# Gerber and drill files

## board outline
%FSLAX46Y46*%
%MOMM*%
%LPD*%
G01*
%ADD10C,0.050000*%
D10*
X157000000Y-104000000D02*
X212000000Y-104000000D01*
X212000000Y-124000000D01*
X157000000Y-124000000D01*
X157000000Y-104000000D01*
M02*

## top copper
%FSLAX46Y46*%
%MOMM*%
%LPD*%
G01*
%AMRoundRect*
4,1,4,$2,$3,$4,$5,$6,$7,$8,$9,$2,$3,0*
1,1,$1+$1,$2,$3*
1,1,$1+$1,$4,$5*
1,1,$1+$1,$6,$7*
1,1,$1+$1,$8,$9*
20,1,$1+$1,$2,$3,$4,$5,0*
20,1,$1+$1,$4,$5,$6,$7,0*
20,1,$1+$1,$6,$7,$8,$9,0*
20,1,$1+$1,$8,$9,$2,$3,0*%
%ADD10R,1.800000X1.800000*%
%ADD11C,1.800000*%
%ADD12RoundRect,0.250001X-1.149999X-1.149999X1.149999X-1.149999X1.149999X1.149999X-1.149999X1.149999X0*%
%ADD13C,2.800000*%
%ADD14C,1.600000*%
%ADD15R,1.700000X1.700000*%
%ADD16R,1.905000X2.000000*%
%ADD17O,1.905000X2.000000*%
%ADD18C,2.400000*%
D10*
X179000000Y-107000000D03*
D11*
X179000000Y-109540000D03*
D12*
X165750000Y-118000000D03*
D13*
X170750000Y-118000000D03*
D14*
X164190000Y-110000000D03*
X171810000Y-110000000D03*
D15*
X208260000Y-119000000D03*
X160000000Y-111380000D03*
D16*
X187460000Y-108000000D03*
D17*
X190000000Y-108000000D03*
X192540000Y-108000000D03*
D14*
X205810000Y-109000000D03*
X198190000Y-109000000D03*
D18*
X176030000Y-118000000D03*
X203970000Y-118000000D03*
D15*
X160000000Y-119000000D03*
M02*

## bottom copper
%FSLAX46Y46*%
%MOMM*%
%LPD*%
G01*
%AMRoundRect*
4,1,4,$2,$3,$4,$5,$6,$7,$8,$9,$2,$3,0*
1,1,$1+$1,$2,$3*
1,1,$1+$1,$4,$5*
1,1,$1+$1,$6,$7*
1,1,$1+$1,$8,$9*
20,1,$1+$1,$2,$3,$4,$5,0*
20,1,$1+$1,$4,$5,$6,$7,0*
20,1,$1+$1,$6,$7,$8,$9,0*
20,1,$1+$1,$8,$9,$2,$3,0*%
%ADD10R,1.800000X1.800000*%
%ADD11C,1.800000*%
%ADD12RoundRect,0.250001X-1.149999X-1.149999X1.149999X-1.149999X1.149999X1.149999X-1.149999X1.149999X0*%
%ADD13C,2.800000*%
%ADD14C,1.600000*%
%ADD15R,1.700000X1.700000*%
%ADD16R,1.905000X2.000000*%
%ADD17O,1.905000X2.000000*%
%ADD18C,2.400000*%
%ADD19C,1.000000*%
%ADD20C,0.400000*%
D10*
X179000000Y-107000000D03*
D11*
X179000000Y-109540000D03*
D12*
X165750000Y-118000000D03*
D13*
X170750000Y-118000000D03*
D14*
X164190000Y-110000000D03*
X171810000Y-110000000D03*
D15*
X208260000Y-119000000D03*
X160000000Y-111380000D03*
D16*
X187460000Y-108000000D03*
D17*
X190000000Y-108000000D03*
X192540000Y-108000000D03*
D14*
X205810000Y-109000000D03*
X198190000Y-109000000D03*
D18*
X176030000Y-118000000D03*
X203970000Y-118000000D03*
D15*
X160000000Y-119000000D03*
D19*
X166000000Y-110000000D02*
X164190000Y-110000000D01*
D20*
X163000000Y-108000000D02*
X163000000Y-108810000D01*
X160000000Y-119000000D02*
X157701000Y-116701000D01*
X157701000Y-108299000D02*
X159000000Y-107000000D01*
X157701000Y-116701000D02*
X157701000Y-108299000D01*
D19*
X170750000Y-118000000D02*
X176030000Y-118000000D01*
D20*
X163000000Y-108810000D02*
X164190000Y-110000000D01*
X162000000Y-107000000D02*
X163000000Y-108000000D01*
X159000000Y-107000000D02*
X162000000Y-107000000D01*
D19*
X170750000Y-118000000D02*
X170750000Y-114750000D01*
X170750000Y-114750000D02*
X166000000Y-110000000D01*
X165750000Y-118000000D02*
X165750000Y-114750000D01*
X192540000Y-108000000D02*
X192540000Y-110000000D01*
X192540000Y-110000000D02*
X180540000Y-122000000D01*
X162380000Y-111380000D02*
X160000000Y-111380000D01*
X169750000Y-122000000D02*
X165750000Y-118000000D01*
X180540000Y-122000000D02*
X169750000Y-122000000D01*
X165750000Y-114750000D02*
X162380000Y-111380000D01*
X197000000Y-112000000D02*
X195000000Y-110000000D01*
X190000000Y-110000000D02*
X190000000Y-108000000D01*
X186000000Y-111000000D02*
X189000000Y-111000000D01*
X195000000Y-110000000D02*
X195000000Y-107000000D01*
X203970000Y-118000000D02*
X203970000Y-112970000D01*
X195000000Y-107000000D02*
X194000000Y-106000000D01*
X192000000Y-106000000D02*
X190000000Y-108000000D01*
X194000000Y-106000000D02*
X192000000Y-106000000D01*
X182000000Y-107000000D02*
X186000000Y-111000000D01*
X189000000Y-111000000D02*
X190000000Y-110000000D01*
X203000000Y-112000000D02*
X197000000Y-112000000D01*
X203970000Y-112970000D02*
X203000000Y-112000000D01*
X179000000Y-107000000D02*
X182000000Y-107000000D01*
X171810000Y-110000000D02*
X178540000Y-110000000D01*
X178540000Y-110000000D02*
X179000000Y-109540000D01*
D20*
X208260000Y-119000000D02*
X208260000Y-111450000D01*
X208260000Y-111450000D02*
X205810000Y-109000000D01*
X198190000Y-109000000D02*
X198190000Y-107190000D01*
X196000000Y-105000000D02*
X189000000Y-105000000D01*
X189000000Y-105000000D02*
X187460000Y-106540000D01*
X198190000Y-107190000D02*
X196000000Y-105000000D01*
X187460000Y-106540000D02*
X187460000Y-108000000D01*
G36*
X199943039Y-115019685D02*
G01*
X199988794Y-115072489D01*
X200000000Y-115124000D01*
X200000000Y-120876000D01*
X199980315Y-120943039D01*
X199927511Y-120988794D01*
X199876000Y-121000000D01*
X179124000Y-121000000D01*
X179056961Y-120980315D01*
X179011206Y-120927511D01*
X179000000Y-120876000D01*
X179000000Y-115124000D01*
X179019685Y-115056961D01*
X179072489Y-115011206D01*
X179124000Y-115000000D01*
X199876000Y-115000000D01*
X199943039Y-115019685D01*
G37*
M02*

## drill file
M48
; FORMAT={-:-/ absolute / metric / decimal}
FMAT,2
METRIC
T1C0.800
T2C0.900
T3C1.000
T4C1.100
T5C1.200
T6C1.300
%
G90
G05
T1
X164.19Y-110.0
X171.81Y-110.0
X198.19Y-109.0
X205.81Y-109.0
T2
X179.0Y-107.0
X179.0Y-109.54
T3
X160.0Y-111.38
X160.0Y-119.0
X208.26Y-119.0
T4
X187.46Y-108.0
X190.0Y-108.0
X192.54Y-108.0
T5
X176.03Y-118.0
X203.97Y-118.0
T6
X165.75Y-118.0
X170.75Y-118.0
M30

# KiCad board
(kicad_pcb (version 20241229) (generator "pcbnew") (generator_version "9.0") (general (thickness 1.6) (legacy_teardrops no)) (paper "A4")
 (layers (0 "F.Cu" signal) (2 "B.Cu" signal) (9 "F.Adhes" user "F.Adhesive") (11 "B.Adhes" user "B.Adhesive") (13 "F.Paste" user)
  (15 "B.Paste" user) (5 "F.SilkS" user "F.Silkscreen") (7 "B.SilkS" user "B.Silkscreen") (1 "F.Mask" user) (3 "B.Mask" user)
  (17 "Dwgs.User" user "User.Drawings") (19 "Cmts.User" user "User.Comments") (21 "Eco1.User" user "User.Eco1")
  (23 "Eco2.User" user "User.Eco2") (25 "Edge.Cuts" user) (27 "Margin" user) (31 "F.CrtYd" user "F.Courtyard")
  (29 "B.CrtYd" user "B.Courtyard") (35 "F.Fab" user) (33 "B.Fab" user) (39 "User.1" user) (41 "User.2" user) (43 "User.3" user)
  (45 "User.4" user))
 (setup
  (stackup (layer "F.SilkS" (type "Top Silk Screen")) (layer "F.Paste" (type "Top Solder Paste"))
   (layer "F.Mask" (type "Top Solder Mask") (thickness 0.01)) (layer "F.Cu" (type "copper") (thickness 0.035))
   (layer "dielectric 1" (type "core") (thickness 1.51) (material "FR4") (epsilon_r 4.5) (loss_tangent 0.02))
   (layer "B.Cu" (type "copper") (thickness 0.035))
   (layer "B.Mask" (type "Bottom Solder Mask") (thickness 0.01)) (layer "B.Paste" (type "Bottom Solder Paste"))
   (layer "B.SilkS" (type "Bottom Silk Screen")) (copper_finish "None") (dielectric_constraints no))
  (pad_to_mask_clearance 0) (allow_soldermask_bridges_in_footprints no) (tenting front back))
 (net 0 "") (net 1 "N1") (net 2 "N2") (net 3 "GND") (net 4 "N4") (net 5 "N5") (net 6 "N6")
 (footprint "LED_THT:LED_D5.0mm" (layer "F.Cu") (at 179 107 -90)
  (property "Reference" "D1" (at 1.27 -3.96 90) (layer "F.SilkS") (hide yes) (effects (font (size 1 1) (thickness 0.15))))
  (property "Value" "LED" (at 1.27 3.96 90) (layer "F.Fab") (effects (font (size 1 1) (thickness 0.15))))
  (pad "1" thru_hole rect (at 0 0 270) (size 1.8 1.8) (drill 0.9) (layers "*.Cu" "*.Mask") (remove_unused_layers no) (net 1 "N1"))
  (pad "2" thru_hole circle (at 2.54 0 270) (size 1.8 1.8) (drill 0.9) (layers "*.Cu" "*.Mask") (remove_unused_layers no) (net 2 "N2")))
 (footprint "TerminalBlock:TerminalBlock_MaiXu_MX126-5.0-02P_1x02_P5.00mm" (layer "F.Cu") (at 165.75 118)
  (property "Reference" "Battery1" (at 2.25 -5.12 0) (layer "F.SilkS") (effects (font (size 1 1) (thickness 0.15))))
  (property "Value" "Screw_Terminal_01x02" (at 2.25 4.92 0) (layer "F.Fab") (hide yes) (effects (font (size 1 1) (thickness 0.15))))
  (pad "1" thru_hole roundrect (at 0 0) (size 2.8 2.8) (drill 1.3) (layers "*.Cu" "*.Mask") (remove_unused_layers no)
   (roundrect_rratio 0.089286) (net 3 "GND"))
  (pad "2" thru_hole circle (at 5 0) (size 2.8 2.8) (drill 1.3) (layers "*.Cu" "*.Mask") (remove_unused_layers no) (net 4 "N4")))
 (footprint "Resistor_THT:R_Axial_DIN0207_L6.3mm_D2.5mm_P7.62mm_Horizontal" (layer "F.Cu") (at 164.19 110)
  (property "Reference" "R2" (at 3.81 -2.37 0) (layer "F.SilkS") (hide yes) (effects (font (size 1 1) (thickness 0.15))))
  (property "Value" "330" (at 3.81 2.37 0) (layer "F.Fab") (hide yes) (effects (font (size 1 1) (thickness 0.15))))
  (pad "1" thru_hole circle (at 0 0) (size 1.6 1.6) (drill 0.8) (layers "*.Cu" "*.Mask") (remove_unused_layers no) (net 4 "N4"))
  (pad "2" thru_hole circle (at 7.62 0) (size 1.6 1.6) (drill 0.8) (layers "*.Cu" "*.Mask") (remove_unused_layers no) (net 2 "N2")))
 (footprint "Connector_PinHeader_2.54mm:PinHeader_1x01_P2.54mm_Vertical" (layer "F.Cu") (at 208.26 119)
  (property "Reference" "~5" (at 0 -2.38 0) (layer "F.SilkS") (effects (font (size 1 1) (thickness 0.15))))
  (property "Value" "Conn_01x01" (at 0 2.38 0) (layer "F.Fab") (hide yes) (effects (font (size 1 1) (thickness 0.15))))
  (pad "1" thru_hole rect (at 0 0) (size 1.7 1.7) (drill 1) (layers "*.Cu" "*.Mask") (remove_unused_layers no) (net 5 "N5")))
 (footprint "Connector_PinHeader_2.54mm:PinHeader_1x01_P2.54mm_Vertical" (layer "F.Cu") (at 160 111.38)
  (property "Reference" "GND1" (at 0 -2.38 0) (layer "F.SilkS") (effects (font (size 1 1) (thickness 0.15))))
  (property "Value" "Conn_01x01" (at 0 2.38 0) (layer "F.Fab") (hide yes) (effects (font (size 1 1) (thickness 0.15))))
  (pad "1" thru_hole rect (at 0 0) (size 1.7 1.7) (drill 1) (layers "*.Cu" "*.Mask") (remove_unused_layers no) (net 3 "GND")))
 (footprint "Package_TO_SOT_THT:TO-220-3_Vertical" (layer "F.Cu") (at 187.46 108)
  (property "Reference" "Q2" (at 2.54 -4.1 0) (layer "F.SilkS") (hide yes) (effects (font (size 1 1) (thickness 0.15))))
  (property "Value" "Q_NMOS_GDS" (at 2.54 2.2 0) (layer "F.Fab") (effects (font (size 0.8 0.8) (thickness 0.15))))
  (pad "1" thru_hole rect (at 0 0) (size 1.905 2) (drill 1.1) (layers "*.Cu" "*.Mask") (remove_unused_layers no) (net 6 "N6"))
  (pad "2" thru_hole oval (at 2.54 0) (size 1.905 2) (drill 1.1) (layers "*.Cu" "*.Mask") (remove_unused_layers no) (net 1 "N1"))
  (pad "3" thru_hole oval (at 5.08 0) (size 1.905 2) (drill 1.1) (layers "*.Cu" "*.Mask") (remove_unused_layers no) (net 3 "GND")))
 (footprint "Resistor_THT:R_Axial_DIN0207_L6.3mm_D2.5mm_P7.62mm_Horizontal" (layer "F.Cu") (at 205.81 109 180)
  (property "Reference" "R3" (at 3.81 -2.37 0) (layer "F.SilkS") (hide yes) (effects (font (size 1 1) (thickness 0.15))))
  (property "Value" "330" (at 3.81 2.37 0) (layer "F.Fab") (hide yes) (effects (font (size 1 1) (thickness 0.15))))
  (pad "1" thru_hole circle (at 0 0 180) (size 1.6 1.6) (drill 0.8) (layers "*.Cu" "*.Mask") (remove_unused_layers no) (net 5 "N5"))
  (pad "2" thru_hole circle (at 7.62 0 180) (size 1.6 1.6) (drill 0.8) (layers "*.Cu" "*.Mask") (remove_unused_layers no) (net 6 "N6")))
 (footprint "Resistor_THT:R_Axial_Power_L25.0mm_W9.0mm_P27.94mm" (layer "F.Cu") (at 176.03 118)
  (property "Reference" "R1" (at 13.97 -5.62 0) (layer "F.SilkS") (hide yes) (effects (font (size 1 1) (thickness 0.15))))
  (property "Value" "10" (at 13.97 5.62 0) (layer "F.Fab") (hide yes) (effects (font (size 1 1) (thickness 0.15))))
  (pad "1" thru_hole circle (at 0 0) (size 2.4 2.4) (drill 1.2) (layers "*.Cu" "*.Mask") (remove_unused_layers no) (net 4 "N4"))
  (pad "2" thru_hole circle (at 27.94 0) (size 2.4 2.4) (drill 1.2) (layers "*.Cu" "*.Mask") (remove_unused_layers no) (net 1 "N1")))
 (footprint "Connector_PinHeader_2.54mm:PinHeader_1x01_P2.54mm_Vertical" (layer "F.Cu") (at 160 119)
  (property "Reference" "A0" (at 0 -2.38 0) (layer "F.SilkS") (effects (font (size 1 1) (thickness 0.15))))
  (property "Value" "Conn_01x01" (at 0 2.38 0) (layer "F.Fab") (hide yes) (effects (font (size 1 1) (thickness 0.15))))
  (pad "1" thru_hole rect (at 0 0) (size 1.7 1.7) (drill 1) (layers "*.Cu" "*.Mask") (remove_unused_layers no) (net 4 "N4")))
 (gr_rect (start 157 104) (end 212 124) (stroke (width 0.05) (type default)) (fill no) (layer "Edge.Cuts"))
 (segment (start 166 110) (end 164.19 110) (width 1) (layer "B.Cu") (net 4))
 (segment (start 163 108) (end 163 108.81) (width 0.4) (layer "B.Cu") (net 4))
 (segment (start 160 119) (end 157.701 116.701) (width 0.4) (layer "B.Cu") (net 4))
 (segment (start 157.701 108.299) (end 159 107) (width 0.4) (layer "B.Cu") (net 4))
 (segment (start 157.701 116.701) (end 157.701 108.299) (width 0.4) (layer "B.Cu") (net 4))
 (segment (start 170.75 118) (end 176.03 118) (width 1) (layer "B.Cu") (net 4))
 (segment (start 163 108.81) (end 164.19 110) (width 0.4) (layer "B.Cu") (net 4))
 (segment (start 162 107) (end 163 108) (width 0.4) (layer "B.Cu") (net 4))
 (segment (start 159 107) (end 162 107) (width 0.4) (layer "B.Cu") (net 4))
 (segment (start 170.75 118) (end 170.75 114.75) (width 1) (layer "B.Cu") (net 4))
 (segment (start 170.75 114.75) (end 166 110) (width 1) (layer "B.Cu") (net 4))
 (segment (start 165.75 118) (end 165.75 114.75) (width 1) (layer "B.Cu") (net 3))
 (segment (start 192.54 108) (end 192.54 110) (width 1) (layer "B.Cu") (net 3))
 (segment (start 192.54 110) (end 180.54 122) (width 1) (layer "B.Cu") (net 3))
 (segment (start 162.38 111.38) (end 160 111.38) (width 1) (layer "B.Cu") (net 3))
 (segment (start 169.75 122) (end 165.75 118) (width 1) (layer "B.Cu") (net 3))
 (segment (start 180.54 122) (end 169.75 122) (width 1) (layer "B.Cu") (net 3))
 (segment (start 165.75 114.75) (end 162.38 111.38) (width 1) (layer "B.Cu") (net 3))
 (segment (start 197 112) (end 195 110) (width 1) (layer "B.Cu") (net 1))
 (segment (start 190 110) (end 190 108) (width 1) (layer "B.Cu") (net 1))
 (segment (start 186 111) (end 189 111) (width 1) (layer "B.Cu") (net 1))
 (segment (start 195 110) (end 195 107) (width 1) (layer "B.Cu") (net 1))
 (segment (start 203.97 118) (end 203.97 112.97) (width 1) (layer "B.Cu") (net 1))
 (segment (start 195 107) (end 194 106) (width 1) (layer "B.Cu") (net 1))
 (segment (start 192 106) (end 190 108) (width 1) (layer "B.Cu") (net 1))
 (segment (start 194 106) (end 192 106) (width 1) (layer "B.Cu") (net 1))
 (segment (start 182 107) (end 186 111) (width 1) (layer "B.Cu") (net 1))
 (segment (start 189 111) (end 190 110) (width 1) (layer "B.Cu") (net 1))
 (segment (start 203 112) (end 197 112) (width 1) (layer "B.Cu") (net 1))
 (segment (start 203.97 112.97) (end 203 112) (width 1) (layer "B.Cu") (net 1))
 (segment (start 179 107) (end 182 107) (width 1) (layer "B.Cu") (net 1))
 (segment (start 171.81 110) (end 178.54 110) (width 1) (layer "B.Cu") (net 2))
 (segment (start 178.54 110) (end 179 109.54) (width 1) (layer "B.Cu") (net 2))
 (segment (start 208.26 119) (end 208.26 111.45) (width 0.4) (layer "B.Cu") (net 5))
 (segment (start 208.26 111.45) (end 205.81 109) (width 0.4) (layer "B.Cu") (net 5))
 (segment (start 198.19 109) (end 198.19 107.19) (width 0.4) (layer "B.Cu") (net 6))
 (segment (start 196 105) (end 189 105) (width 0.4) (layer "B.Cu") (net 6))
 (segment (start 189 105) (end 187.46 106.54) (width 0.4) (layer "B.Cu") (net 6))
 (segment (start 198.19 107.19) (end 196 105) (width 0.4) (layer "B.Cu") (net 6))
 (segment (start 187.46 106.54) (end 187.46 108) (width 0.4) (layer "B.Cu") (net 6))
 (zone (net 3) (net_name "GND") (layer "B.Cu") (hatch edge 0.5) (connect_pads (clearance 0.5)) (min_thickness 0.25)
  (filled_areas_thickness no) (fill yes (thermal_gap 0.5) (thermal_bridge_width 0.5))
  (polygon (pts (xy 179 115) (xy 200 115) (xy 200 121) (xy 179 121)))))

